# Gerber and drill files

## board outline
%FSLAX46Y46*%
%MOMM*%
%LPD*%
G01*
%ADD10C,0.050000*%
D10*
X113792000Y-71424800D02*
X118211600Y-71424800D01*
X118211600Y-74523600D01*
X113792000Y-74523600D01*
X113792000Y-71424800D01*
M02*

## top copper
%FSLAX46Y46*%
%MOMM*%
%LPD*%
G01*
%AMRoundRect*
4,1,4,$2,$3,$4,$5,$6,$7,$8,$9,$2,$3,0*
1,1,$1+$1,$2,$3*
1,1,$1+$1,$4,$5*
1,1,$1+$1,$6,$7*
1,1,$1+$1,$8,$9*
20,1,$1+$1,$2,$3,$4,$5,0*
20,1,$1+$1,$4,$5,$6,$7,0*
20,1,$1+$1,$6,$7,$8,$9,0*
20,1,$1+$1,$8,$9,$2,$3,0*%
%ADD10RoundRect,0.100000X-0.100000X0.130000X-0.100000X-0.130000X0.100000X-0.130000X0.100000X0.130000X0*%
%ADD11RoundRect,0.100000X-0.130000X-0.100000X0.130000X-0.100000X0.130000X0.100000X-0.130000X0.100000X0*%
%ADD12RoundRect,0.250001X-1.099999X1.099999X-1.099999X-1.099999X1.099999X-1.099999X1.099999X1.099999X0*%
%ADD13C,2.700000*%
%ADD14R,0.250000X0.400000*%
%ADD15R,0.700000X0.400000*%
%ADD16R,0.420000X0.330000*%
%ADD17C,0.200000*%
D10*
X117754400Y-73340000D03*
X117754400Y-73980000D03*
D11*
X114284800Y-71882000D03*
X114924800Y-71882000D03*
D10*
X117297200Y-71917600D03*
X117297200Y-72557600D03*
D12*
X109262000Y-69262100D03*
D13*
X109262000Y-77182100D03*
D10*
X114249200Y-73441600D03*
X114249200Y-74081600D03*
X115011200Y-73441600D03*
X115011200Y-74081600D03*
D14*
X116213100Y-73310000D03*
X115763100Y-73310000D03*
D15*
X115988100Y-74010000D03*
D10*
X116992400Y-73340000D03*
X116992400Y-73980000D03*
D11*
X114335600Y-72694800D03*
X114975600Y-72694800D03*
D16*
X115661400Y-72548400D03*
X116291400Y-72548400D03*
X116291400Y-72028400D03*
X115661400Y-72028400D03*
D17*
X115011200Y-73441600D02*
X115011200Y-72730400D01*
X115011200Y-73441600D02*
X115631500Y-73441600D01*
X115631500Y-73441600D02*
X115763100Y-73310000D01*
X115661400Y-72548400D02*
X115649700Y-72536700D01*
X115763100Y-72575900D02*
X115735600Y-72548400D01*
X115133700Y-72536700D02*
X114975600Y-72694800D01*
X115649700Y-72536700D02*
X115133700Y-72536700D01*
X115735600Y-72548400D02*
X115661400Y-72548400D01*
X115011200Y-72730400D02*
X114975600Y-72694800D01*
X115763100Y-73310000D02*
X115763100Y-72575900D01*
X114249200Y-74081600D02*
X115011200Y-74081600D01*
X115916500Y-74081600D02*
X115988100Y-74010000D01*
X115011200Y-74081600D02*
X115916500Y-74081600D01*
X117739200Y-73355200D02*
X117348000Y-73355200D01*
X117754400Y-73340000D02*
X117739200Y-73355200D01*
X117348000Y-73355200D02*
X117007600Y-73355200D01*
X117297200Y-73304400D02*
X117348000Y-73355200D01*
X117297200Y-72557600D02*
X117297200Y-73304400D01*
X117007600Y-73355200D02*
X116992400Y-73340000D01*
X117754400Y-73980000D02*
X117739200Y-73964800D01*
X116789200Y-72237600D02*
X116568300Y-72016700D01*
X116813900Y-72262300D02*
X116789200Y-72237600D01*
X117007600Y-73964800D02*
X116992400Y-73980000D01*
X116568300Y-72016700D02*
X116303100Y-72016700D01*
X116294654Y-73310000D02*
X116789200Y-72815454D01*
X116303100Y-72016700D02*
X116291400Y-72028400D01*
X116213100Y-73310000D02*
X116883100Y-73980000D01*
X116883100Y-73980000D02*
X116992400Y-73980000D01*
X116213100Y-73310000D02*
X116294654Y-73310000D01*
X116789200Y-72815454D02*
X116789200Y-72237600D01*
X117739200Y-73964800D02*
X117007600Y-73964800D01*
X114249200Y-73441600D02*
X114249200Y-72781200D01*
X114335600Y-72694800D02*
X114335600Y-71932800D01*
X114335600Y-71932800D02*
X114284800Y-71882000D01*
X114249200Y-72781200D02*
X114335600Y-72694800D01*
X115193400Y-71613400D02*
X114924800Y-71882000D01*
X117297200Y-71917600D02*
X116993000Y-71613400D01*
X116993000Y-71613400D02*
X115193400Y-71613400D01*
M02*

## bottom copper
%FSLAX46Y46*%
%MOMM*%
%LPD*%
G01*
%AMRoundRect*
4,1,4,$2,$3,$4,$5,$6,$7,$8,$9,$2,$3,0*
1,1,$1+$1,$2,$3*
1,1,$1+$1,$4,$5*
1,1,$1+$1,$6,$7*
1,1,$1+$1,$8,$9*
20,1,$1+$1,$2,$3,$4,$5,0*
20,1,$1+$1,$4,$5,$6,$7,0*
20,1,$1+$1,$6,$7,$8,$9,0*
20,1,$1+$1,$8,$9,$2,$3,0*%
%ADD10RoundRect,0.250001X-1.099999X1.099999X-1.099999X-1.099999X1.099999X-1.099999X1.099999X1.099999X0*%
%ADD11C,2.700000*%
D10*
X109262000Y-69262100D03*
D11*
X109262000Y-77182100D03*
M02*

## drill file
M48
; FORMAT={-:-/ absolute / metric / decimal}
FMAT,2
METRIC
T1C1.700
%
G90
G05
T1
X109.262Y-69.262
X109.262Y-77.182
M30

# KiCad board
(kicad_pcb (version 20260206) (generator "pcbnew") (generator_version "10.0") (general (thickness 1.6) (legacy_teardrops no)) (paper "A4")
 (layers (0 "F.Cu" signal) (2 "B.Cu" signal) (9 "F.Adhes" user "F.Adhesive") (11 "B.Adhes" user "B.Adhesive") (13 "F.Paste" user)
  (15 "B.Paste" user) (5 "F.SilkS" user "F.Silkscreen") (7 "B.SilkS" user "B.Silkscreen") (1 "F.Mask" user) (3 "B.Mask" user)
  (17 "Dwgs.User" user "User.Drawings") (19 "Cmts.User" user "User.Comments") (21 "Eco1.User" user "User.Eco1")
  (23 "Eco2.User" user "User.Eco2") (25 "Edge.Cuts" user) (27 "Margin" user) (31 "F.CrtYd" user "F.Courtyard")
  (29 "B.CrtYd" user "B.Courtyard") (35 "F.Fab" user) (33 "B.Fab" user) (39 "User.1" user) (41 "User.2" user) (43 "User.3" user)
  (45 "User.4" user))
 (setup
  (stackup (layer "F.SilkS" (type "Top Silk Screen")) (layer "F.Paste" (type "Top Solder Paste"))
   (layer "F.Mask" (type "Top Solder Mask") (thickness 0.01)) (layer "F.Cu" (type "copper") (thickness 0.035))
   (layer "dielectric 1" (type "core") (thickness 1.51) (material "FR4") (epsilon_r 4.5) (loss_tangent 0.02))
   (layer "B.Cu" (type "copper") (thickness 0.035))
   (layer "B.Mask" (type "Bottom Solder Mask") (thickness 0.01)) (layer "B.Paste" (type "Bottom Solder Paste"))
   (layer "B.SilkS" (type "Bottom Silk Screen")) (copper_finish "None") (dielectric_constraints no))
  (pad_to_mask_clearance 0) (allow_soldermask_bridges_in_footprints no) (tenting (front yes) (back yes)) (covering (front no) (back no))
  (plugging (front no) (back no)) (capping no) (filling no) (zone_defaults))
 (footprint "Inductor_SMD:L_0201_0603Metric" (layer "F.Cu") (at 117.7544 73.66 -90)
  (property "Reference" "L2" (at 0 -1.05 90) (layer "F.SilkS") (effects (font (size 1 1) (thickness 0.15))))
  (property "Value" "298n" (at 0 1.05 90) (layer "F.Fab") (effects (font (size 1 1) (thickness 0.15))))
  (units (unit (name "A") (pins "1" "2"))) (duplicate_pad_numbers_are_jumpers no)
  (pad "" smd roundrect (at -0.345 0 270) (size 0.318 0.36) (layers "F.Paste") (roundrect_rratio 0.25))
  (pad "" smd roundrect (at 0.345 0 270) (size 0.318 0.36) (layers "F.Paste") (roundrect_rratio 0.25))
  (pad "1" smd roundrect (at -0.32 0 270) (size 0.46 0.4) (layers "F.Cu" "F.Mask") (roundrect_rratio 0.25) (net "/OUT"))
  (pad "2" smd roundrect (at 0.32 0 270) (size 0.46 0.4) (layers "F.Cu" "F.Mask") (roundrect_rratio 0.25) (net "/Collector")))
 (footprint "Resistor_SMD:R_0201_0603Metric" (layer "F.Cu") (at 114.6048 71.882)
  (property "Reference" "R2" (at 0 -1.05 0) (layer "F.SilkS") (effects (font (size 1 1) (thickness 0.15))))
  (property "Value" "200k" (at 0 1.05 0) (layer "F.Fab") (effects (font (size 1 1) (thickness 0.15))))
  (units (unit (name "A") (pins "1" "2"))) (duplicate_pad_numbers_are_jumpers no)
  (pad "" smd roundrect (at -0.345 0) (size 0.318 0.36) (layers "F.Paste") (roundrect_rratio 0.25))
  (pad "" smd roundrect (at 0.345 0) (size 0.318 0.36) (layers "F.Paste") (roundrect_rratio 0.25))
  (pad "1" smd roundrect (at -0.32 0) (size 0.46 0.4) (layers "F.Cu" "F.Mask") (roundrect_rratio 0.25) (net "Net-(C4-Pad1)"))
  (pad "2" smd roundrect (at 0.32 0) (size 0.46 0.4) (layers "F.Cu" "F.Mask") (roundrect_rratio 0.25) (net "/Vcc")))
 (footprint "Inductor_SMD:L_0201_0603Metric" (layer "F.Cu") (at 117.2972 72.2376 -90)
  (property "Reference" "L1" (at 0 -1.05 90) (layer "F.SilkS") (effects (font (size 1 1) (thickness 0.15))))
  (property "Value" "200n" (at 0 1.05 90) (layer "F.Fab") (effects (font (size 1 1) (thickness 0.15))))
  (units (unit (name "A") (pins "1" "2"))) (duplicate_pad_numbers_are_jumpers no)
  (pad "" smd roundrect (at -0.345 0 270) (size 0.318 0.36) (layers "F.Paste") (roundrect_rratio 0.25))
  (pad "" smd roundrect (at 0.345 0 270) (size 0.318 0.36) (layers "F.Paste") (roundrect_rratio 0.25))
  (pad "1" smd roundrect (at -0.32 0 270) (size 0.46 0.4) (layers "F.Cu" "F.Mask") (roundrect_rratio 0.25) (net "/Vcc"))
  (pad "2" smd roundrect (at 0.32 0 270) (size 0.46 0.4) (layers "F.Cu" "F.Mask") (roundrect_rratio 0.25) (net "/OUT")))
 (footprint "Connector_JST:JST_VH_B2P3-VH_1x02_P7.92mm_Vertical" (layer "F.Cu") (at 109.262 69.2621 -90)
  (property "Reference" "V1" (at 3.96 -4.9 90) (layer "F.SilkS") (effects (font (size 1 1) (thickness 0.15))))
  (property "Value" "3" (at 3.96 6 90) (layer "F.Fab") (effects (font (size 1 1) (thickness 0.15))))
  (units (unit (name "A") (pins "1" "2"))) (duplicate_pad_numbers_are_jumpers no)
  (pad "1" thru_hole roundrect (at 0 0 270) (size 2.7 2.7) (drill 1.7) (layers "*.Cu" "*.Mask") (remove_unused_layers no)
   (roundrect_rratio 0.092593) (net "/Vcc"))
  (pad "2" thru_hole circle (at 7.92 0 270) (size 2.7 2.7) (drill 1.7) (layers "*.Cu" "*.Mask") (remove_unused_layers no) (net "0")))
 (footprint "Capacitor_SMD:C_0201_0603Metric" (layer "F.Cu") (at 114.2492 73.7616 -90)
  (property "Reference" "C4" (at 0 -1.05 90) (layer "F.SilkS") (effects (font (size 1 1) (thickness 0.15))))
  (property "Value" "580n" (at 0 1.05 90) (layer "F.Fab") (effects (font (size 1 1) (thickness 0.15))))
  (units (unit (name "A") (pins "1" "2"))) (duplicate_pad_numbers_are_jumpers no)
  (pad "" smd roundrect (at -0.345 0 270) (size 0.318 0.36) (layers "F.Paste") (roundrect_rratio 0.25))
  (pad "" smd roundrect (at 0.345 0 270) (size 0.318 0.36) (layers "F.Paste") (roundrect_rratio 0.25))
  (pad "1" smd roundrect (at -0.32 0 270) (size 0.46 0.4) (layers "F.Cu" "F.Mask") (roundrect_rratio 0.25) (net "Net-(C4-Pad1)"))
  (pad "2" smd roundrect (at 0.32 0 270) (size 0.46 0.4) (layers "F.Cu" "F.Mask") (roundrect_rratio 0.25) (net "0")))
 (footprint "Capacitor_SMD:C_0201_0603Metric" (layer "F.Cu") (at 115.0112 73.7616 -90)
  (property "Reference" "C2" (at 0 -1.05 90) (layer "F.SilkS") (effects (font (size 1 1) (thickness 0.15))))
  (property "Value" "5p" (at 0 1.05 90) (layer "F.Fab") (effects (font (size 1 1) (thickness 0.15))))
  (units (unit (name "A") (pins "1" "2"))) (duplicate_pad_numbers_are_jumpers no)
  (pad "" smd roundrect (at -0.345 0 270) (size 0.318 0.36) (layers "F.Paste") (roundrect_rratio 0.25))
  (pad "" smd roundrect (at 0.345 0 270) (size 0.318 0.36) (layers "F.Paste") (roundrect_rratio 0.25))
  (pad "1" smd roundrect (at -0.32 0 270) (size 0.46 0.4) (layers "F.Cu" "F.Mask") (roundrect_rratio 0.25) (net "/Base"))
  (pad "2" smd roundrect (at 0.32 0 270) (size 0.46 0.4) (layers "F.Cu" "F.Mask") (roundrect_rratio 0.25) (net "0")))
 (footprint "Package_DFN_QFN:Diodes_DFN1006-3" (layer "F.Cu") (at 115.9881 73.66 -90)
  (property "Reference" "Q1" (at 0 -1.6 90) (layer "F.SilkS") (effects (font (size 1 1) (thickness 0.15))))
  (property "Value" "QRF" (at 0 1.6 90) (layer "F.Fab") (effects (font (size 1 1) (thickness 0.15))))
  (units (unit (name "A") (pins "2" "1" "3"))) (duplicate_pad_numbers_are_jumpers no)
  (pad "1" smd rect (at -0.35 -0.225 180) (size 0.25 0.4) (layers "F.Cu" "F.Mask" "F.Paste") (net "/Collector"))
  (pad "2" smd rect (at -0.35 0.225 180) (size 0.25 0.4) (layers "F.Cu" "F.Mask" "F.Paste") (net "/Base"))
  (pad "3" smd rect (at 0.35 0 180) (size 0.7 0.4) (layers "F.Cu" "F.Mask" "F.Paste") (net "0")))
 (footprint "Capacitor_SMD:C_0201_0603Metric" (layer "F.Cu") (at 116.9924 73.66 -90)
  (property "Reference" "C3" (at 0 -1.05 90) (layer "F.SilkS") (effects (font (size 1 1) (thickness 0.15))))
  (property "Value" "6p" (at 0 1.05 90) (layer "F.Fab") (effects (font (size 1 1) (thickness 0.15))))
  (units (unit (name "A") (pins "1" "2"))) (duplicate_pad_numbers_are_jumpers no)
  (pad "" smd roundrect (at -0.345 0 270) (size 0.318 0.36) (layers "F.Paste") (roundrect_rratio 0.25))
  (pad "" smd roundrect (at 0.345 0 270) (size 0.318 0.36) (layers "F.Paste") (roundrect_rratio 0.25))
  (pad "1" smd roundrect (at -0.32 0 270) (size 0.46 0.4) (layers "F.Cu" "F.Mask") (roundrect_rratio 0.25) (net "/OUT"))
  (pad "2" smd roundrect (at 0.32 0 270) (size 0.46 0.4) (layers "F.Cu" "F.Mask") (roundrect_rratio 0.25) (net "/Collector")))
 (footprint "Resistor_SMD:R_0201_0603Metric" (layer "F.Cu") (at 114.6556 72.6948)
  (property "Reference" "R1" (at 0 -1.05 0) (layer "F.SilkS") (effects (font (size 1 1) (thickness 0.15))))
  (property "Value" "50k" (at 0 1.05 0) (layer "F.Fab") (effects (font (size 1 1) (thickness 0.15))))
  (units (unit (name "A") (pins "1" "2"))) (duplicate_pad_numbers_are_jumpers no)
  (pad "" smd roundrect (at -0.345 0) (size 0.318 0.36) (layers "F.Paste") (roundrect_rratio 0.25))
  (pad "" smd roundrect (at 0.345 0) (size 0.318 0.36) (layers "F.Paste") (roundrect_rratio 0.25))
  (pad "1" smd roundrect (at -0.32 0) (size 0.46 0.4) (layers "F.Cu" "F.Mask") (roundrect_rratio 0.25) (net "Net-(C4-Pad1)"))
  (pad "2" smd roundrect (at 0.32 0) (size 0.46 0.4) (layers "F.Cu" "F.Mask") (roundrect_rratio 0.25) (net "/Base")))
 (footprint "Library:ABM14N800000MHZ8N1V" (layer "F.Cu") (at 115.9764 72.2884)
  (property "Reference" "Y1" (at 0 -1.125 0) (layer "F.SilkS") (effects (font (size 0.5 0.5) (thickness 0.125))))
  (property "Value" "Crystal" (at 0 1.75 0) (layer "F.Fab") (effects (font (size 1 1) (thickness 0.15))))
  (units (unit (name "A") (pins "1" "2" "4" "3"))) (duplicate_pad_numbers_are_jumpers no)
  (pad "1" smd rect (at -0.315 0.26) (size 0.42 0.33) (layers "F.Cu" "F.Mask" "F.Paste") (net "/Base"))
  (pad "2" smd rect (at 0.315 0.26) (size 0.42 0.33) (layers "F.Cu" "F.Mask" "F.Paste") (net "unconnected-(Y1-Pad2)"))
  (pad "3" smd rect (at 0.315 -0.26) (size 0.42 0.33) (layers "F.Cu" "F.Mask" "F.Paste") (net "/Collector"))
  (pad "4" smd rect (at -0.315 -0.26) (size 0.42 0.33) (layers "F.Cu" "F.Mask" "F.Paste") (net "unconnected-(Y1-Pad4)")))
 (gr_rect (start 113.792 71.4248) (end 118.2116 74.5236) (stroke (width 0.05) (type default)) (fill no) (layer "Edge.Cuts"))
 (segment (start 115.0112 73.4416) (end 115.0112 72.7304) (width 0.2) (layer "F.Cu") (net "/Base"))
 (segment (start 115.0112 73.4416) (end 115.6315 73.4416) (width 0.2) (layer "F.Cu") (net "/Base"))
 (segment (start 115.6315 73.4416) (end 115.7631 73.31) (width 0.2) (layer "F.Cu") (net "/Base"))
 (segment (start 115.6614 72.5484) (end 115.6497 72.5367) (width 0.2) (layer "F.Cu") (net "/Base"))
 (segment (start 115.7631 72.5759) (end 115.7356 72.5484) (width 0.2) (layer "F.Cu") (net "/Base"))
 (segment (start 115.1337 72.5367) (end 114.9756 72.6948) (width 0.2) (layer "F.Cu") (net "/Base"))
 (segment (start 115.6497 72.5367) (end 115.1337 72.5367) (width 0.2) (layer "F.Cu") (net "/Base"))
 (segment (start 115.7356 72.5484) (end 115.6614 72.5484) (width 0.2) (layer "F.Cu") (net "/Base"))
 (segment (start 115.0112 72.7304) (end 114.9756 72.6948) (width 0.2) (layer "F.Cu") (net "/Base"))
 (segment (start 115.7631 73.31) (end 115.7631 72.5759) (width 0.2) (layer "F.Cu") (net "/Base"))
 (segment (start 114.2492 74.0816) (end 115.0112 74.0816) (width 0.2) (layer "F.Cu") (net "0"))
 (segment (start 115.9165 74.0816) (end 115.9881 74.01) (width 0.2) (layer "F.Cu") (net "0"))
 (segment (start 115.0112 74.0816) (end 115.9165 74.0816) (width 0.2) (layer "F.Cu") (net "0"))
 (segment (start 117.7392 73.3552) (end 117.348 73.3552) (width 0.2) (layer "F.Cu") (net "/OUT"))
 (segment (start 117.7544 73.34) (end 117.7392 73.3552) (width 0.2) (layer "F.Cu") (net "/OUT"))
 (segment (start 117.348 73.3552) (end 117.0076 73.3552) (width 0.2) (layer "F.Cu") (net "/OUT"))
 (segment (start 117.2972 73.3044) (end 117.348 73.3552) (width 0.2) (layer "F.Cu") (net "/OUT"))
 (segment (start 117.2972 72.5576) (end 117.2972 73.3044) (width 0.2) (layer "F.Cu") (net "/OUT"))
 (segment (start 117.0076 73.3552) (end 116.9924 73.34) (width 0.2) (layer "F.Cu") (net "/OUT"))
 (segment (start 117.7544 73.98) (end 117.7392 73.9648) (width 0.2) (layer "F.Cu") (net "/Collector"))
 (segment (start 116.7892 72.2376) (end 116.5683 72.0167) (width 0.2) (layer "F.Cu") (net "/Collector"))
 (segment (start 116.8139 72.2623) (end 116.7892 72.2376) (width 0.2) (layer "F.Cu") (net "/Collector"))
 (segment (start 117.0076 73.9648) (end 116.9924 73.98) (width 0.2) (layer "F.Cu") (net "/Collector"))
 (segment (start 116.5683 72.0167) (end 116.3031 72.0167) (width 0.2) (layer "F.Cu") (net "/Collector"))
 (segment (start 116.294654 73.31) (end 116.7892 72.815454) (width 0.2) (layer "F.Cu") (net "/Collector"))
 (segment (start 116.3031 72.0167) (end 116.2914 72.0284) (width 0.2) (layer "F.Cu") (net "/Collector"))
 (segment (start 116.2131 73.31) (end 116.8831 73.98) (width 0.2) (layer "F.Cu") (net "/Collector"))
 (segment (start 116.8831 73.98) (end 116.9924 73.98) (width 0.2) (layer "F.Cu") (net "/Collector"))
 (segment (start 116.2131 73.31) (end 116.294654 73.31) (width 0.2) (layer "F.Cu") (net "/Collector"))
 (segment (start 116.7892 72.815454) (end 116.7892 72.2376) (width 0.2) (layer "F.Cu") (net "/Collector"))
 (segment (start 117.7392 73.9648) (end 117.0076 73.9648) (width 0.2) (layer "F.Cu") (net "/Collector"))
 (segment (start 114.2492 73.4416) (end 114.2492 72.7812) (width 0.2) (layer "F.Cu") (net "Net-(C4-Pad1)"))
 (segment (start 114.3356 72.6948) (end 114.3356 71.9328) (width 0.2) (layer "F.Cu") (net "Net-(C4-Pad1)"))
 (segment (start 114.3356 71.9328) (end 114.2848 71.882) (width 0.2) (layer "F.Cu") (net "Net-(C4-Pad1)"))
 (segment (start 114.2492 72.7812) (end 114.3356 72.6948) (width 0.2) (layer "F.Cu") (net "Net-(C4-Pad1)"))
 (segment (start 115.1934 71.6134) (end 114.9248 71.882) (width 0.2) (layer "F.Cu") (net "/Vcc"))
 (segment (start 117.2972 71.9176) (end 116.993 71.6134) (width 0.2) (layer "F.Cu") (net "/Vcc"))
 (segment (start 116.993 71.6134) (end 115.1934 71.6134) (width 0.2) (layer "F.Cu") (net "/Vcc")))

